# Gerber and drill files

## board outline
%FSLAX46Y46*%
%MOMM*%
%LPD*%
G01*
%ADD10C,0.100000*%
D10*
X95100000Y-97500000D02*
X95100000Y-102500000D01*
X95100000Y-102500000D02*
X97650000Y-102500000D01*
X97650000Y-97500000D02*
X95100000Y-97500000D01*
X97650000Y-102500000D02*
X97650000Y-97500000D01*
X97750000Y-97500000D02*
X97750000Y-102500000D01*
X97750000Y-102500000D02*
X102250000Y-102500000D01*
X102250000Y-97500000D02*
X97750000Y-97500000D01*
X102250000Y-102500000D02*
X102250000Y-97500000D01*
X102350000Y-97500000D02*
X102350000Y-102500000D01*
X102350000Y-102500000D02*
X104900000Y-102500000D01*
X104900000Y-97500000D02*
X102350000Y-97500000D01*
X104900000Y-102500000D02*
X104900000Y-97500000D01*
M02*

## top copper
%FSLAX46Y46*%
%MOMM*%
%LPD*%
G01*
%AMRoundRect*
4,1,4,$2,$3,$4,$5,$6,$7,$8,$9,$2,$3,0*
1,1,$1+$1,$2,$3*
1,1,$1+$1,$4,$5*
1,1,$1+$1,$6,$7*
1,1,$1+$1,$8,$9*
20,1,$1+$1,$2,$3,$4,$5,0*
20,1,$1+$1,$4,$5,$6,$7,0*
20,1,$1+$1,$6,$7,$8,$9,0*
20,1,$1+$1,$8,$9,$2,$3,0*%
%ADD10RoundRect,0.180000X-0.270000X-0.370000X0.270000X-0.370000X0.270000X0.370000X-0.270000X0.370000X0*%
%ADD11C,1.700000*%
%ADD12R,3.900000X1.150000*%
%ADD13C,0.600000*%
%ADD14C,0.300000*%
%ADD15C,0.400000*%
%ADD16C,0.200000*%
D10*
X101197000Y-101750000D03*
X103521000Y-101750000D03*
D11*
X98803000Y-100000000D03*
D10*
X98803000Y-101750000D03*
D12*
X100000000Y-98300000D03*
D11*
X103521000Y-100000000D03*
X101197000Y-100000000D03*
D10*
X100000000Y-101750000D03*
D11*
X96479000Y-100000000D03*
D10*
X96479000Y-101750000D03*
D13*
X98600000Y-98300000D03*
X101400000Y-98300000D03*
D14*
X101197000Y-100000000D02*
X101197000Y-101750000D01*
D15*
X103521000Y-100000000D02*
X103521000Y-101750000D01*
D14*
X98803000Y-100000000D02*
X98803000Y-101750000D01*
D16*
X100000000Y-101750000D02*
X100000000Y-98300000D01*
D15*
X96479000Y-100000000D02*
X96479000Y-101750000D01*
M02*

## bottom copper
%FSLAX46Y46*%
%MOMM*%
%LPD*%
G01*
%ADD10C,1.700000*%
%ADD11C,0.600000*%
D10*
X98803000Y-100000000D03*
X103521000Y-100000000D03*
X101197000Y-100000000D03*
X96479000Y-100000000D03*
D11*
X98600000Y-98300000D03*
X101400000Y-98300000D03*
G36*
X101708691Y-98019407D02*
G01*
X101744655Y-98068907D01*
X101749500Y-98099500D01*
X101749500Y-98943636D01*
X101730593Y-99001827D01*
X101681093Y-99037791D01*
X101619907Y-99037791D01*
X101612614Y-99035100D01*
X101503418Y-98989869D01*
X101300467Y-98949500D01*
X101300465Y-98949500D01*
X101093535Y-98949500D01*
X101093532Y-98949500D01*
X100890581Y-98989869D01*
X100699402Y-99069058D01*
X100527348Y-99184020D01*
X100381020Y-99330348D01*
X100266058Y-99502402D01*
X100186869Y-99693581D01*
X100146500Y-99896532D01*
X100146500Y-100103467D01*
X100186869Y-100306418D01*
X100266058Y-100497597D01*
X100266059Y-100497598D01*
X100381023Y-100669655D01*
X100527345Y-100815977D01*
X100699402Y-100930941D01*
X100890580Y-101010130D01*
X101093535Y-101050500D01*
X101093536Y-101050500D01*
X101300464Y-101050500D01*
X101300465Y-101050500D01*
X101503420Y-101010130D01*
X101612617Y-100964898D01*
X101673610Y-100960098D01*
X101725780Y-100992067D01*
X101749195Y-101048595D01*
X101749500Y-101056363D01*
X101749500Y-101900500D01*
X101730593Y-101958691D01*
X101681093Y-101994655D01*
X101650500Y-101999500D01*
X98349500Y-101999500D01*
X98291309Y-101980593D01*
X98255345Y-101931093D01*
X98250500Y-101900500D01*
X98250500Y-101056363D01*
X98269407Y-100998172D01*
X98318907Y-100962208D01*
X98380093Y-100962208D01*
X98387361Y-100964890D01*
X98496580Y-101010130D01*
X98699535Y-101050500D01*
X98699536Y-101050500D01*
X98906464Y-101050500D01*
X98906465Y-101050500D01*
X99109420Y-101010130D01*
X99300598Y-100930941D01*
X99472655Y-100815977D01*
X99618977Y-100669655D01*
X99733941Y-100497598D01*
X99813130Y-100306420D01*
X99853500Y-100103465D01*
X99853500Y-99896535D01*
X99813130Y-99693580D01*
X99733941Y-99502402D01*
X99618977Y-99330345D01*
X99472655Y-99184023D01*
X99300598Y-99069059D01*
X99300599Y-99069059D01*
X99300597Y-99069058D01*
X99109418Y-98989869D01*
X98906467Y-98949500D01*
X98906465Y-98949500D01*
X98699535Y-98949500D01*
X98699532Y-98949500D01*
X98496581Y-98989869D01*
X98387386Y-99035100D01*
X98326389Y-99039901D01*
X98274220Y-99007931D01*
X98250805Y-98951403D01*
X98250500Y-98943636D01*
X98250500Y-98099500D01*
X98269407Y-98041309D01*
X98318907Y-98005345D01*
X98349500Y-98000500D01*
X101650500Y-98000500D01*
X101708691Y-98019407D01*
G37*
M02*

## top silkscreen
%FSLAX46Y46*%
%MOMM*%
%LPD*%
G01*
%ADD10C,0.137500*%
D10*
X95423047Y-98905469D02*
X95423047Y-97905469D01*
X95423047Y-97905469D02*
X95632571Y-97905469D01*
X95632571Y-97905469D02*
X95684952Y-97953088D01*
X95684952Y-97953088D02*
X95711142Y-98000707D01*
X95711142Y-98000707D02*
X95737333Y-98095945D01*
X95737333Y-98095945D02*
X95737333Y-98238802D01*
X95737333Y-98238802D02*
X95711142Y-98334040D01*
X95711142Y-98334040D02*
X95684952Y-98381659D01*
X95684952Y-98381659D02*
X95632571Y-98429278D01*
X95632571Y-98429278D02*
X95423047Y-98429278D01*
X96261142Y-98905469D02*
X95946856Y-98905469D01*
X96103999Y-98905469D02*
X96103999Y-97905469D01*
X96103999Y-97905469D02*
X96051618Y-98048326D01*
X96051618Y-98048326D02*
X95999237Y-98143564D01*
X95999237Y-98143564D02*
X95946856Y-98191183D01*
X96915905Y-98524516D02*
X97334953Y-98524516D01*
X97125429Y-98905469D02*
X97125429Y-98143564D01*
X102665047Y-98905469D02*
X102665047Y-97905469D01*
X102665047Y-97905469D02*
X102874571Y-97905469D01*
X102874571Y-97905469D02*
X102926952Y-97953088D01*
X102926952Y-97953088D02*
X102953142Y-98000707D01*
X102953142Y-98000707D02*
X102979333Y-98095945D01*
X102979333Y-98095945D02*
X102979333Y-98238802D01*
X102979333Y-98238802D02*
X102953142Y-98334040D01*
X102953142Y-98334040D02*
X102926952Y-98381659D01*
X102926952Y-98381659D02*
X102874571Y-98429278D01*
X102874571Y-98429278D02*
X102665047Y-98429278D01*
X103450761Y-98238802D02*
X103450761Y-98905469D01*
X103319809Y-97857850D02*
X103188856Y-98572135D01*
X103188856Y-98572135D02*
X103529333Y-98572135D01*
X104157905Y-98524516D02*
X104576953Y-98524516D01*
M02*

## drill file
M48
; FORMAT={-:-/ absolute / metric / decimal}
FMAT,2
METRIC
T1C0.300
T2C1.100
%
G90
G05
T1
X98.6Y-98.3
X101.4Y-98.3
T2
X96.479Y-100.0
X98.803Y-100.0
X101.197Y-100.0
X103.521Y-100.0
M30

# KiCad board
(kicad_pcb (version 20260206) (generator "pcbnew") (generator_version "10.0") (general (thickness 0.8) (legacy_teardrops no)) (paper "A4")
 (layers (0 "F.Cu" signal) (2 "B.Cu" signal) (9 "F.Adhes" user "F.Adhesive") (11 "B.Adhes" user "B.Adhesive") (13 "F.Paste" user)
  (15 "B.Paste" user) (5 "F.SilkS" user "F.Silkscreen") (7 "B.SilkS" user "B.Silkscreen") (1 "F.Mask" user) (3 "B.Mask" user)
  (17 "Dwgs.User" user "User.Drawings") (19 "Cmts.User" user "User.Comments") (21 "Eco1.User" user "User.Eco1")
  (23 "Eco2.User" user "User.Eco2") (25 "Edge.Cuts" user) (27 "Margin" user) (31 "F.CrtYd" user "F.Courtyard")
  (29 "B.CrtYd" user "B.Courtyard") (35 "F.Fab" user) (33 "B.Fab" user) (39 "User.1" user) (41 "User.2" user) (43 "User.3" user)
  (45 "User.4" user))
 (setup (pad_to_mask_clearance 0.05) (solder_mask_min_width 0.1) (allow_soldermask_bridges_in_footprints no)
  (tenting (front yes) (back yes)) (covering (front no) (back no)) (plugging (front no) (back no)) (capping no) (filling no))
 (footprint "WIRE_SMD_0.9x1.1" (layer "F.Cu") (at 101.197 101.75)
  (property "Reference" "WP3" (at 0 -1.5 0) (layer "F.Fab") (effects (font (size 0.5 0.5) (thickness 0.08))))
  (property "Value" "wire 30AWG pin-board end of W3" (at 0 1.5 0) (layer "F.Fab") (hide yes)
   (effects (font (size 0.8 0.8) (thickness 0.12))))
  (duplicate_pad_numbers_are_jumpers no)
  (pad "1" smd roundrect (at 0 0) (size 0.9 1.1) (layers "F.Cu" "F.Mask") (roundrect_rratio 0.2) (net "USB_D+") (thermal_bridge_angle 45)))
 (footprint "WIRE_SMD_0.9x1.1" (layer "F.Cu") (at 103.521 101.75)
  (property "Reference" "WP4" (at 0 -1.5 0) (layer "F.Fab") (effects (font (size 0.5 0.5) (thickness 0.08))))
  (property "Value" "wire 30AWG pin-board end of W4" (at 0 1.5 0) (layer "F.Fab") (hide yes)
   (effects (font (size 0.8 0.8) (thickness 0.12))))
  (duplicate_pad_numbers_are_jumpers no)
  (pad "1" smd roundrect (at 0 0) (size 0.9 1.1) (layers "F.Cu" "F.Mask") (roundrect_rratio 0.2) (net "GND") (thermal_bridge_angle 45)))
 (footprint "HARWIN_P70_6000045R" (layer "F.Cu") (at 98.803 100)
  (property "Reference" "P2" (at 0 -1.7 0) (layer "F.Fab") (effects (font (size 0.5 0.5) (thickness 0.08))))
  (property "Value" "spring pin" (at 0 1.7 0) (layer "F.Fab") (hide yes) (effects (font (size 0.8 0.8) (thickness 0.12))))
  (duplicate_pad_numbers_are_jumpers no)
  (pad "1" thru_hole circle (at 0 0) (size 1.7 1.7) (drill 1.1) (layers "*.Cu" "*.Mask") (remove_unused_layers no) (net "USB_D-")))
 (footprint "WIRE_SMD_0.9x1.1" (layer "F.Cu") (at 98.803 101.75)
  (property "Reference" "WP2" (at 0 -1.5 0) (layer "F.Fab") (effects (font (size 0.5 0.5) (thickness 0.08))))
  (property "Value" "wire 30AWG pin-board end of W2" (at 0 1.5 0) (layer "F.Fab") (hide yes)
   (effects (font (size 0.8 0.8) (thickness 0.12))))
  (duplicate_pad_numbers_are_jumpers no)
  (pad "1" smd roundrect (at 0 0) (size 0.9 1.1) (layers "F.Cu" "F.Mask") (roundrect_rratio 0.2) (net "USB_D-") (thermal_bridge_angle 45)))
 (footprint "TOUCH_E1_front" (layer "F.Cu") (at 100 98.3)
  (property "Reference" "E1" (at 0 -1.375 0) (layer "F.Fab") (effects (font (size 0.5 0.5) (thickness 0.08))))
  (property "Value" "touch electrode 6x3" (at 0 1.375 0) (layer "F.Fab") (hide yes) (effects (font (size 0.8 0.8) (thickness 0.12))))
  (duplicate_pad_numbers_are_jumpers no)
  (pad "1" smd rect (at 0 0) (size 3.9 1.15) (layers "F.Cu" "F.Mask") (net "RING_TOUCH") (thermal_bridge_angle 45)))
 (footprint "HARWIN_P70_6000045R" (layer "F.Cu") (at 103.521 100)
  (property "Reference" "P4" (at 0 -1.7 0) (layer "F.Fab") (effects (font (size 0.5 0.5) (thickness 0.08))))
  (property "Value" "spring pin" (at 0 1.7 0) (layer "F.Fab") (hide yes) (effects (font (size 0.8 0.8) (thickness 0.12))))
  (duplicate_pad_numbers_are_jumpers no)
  (pad "1" thru_hole circle (at 0 0) (size 1.7 1.7) (drill 1.1) (layers "*.Cu" "*.Mask") (remove_unused_layers no) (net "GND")))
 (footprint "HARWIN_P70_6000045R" (layer "F.Cu") (at 101.197 100)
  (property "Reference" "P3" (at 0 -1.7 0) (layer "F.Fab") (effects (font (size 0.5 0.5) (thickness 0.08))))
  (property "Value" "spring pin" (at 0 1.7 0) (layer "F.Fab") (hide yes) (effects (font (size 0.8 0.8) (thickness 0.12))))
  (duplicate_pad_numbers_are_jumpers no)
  (pad "1" thru_hole circle (at 0 0) (size 1.7 1.7) (drill 1.1) (layers "*.Cu" "*.Mask") (remove_unused_layers no) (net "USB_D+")))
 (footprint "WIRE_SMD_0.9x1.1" (layer "F.Cu") (at 100 101.75)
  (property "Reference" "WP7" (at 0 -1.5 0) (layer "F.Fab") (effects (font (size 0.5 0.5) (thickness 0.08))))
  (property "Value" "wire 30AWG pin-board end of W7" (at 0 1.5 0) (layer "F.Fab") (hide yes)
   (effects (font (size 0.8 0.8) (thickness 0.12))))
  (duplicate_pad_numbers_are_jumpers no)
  (pad "1" smd roundrect (at 0 0) (size 0.9 1.1) (layers "F.Cu" "F.Mask") (roundrect_rratio 0.2) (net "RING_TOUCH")
   (thermal_bridge_angle 45)))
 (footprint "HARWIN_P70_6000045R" (layer "F.Cu") (at 96.479 100)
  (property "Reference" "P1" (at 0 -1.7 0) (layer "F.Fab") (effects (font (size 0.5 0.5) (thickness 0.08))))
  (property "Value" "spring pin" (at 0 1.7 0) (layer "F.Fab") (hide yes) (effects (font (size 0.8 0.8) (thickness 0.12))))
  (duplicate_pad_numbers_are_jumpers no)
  (pad "1" thru_hole circle (at 0 0) (size 1.7 1.7) (drill 1.1) (layers "*.Cu" "*.Mask") (remove_unused_layers no) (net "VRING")))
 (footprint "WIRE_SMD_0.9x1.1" (layer "F.Cu") (at 96.479 101.75)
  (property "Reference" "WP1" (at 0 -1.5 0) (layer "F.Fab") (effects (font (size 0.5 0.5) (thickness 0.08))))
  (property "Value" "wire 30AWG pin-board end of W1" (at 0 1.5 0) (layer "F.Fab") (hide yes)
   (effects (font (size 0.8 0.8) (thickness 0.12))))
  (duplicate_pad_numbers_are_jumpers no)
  (pad "1" smd roundrect (at 0 0) (size 0.9 1.1) (layers "F.Cu" "F.Mask") (roundrect_rratio 0.2) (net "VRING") (thermal_bridge_angle 45)))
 (gr_line (start 95.1 97.5) (end 95.1 102.5) (stroke (width 0.1) (type default)) (layer "Edge.Cuts"))
 (gr_line (start 95.1 102.5) (end 97.65 102.5) (stroke (width 0.1) (type default)) (layer "Edge.Cuts"))
 (gr_line (start 97.65 97.5) (end 95.1 97.5) (stroke (width 0.1) (type default)) (layer "Edge.Cuts"))
 (gr_line (start 97.65 102.5) (end 97.65 97.5) (stroke (width 0.1) (type default)) (layer "Edge.Cuts"))
 (gr_line (start 97.75 97.5) (end 97.75 102.5) (stroke (width 0.1) (type default)) (layer "Edge.Cuts"))
 (gr_line (start 97.75 102.5) (end 102.25 102.5) (stroke (width 0.1) (type default)) (layer "Edge.Cuts"))
 (gr_line (start 102.25 97.5) (end 97.75 97.5) (stroke (width 0.1) (type default)) (layer "Edge.Cuts"))
 (gr_line (start 102.25 102.5) (end 102.25 97.5) (stroke (width 0.1) (type default)) (layer "Edge.Cuts"))
 (gr_line (start 102.35 97.5) (end 102.35 102.5) (stroke (width 0.1) (type default)) (layer "Edge.Cuts"))
 (gr_line (start 102.35 102.5) (end 104.9 102.5) (stroke (width 0.1) (type default)) (layer "Edge.Cuts"))
 (gr_line (start 104.9 97.5) (end 102.35 97.5) (stroke (width 0.1) (type default)) (layer "Edge.Cuts"))
 (gr_line (start 104.9 102.5) (end 104.9 97.5) (stroke (width 0.1) (type default)) (layer "Edge.Cuts"))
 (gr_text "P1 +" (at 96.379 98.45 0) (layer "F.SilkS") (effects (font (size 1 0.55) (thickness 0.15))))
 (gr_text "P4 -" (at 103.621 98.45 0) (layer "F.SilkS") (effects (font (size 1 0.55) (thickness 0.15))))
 (segment (start 101.197 100) (end 101.197 101.75) (width 0.3) (layer "F.Cu") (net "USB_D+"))
 (segment (start 103.521 100) (end 103.521 101.75) (width 0.4) (layer "F.Cu") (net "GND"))
 (segment (start 98.803 100) (end 98.803 101.75) (width 0.3) (layer "F.Cu") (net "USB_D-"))
 (segment (start 100 101.75) (end 100 98.3) (width 0.2) (layer "F.Cu") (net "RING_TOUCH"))
 (via (at 98.6 98.3) (size 0.6) (drill 0.3) (layers "F.Cu" "B.Cu") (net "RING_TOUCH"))
 (via (at 101.4 98.3) (size 0.6) (drill 0.3) (layers "F.Cu" "B.Cu") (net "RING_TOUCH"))
 (segment (start 96.479 100) (end 96.479 101.75) (width 0.4) (layer "F.Cu") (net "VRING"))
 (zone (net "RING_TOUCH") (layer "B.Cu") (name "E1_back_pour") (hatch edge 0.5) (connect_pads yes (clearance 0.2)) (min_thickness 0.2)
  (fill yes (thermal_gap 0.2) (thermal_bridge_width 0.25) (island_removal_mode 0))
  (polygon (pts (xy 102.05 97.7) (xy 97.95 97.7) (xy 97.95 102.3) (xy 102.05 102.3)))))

